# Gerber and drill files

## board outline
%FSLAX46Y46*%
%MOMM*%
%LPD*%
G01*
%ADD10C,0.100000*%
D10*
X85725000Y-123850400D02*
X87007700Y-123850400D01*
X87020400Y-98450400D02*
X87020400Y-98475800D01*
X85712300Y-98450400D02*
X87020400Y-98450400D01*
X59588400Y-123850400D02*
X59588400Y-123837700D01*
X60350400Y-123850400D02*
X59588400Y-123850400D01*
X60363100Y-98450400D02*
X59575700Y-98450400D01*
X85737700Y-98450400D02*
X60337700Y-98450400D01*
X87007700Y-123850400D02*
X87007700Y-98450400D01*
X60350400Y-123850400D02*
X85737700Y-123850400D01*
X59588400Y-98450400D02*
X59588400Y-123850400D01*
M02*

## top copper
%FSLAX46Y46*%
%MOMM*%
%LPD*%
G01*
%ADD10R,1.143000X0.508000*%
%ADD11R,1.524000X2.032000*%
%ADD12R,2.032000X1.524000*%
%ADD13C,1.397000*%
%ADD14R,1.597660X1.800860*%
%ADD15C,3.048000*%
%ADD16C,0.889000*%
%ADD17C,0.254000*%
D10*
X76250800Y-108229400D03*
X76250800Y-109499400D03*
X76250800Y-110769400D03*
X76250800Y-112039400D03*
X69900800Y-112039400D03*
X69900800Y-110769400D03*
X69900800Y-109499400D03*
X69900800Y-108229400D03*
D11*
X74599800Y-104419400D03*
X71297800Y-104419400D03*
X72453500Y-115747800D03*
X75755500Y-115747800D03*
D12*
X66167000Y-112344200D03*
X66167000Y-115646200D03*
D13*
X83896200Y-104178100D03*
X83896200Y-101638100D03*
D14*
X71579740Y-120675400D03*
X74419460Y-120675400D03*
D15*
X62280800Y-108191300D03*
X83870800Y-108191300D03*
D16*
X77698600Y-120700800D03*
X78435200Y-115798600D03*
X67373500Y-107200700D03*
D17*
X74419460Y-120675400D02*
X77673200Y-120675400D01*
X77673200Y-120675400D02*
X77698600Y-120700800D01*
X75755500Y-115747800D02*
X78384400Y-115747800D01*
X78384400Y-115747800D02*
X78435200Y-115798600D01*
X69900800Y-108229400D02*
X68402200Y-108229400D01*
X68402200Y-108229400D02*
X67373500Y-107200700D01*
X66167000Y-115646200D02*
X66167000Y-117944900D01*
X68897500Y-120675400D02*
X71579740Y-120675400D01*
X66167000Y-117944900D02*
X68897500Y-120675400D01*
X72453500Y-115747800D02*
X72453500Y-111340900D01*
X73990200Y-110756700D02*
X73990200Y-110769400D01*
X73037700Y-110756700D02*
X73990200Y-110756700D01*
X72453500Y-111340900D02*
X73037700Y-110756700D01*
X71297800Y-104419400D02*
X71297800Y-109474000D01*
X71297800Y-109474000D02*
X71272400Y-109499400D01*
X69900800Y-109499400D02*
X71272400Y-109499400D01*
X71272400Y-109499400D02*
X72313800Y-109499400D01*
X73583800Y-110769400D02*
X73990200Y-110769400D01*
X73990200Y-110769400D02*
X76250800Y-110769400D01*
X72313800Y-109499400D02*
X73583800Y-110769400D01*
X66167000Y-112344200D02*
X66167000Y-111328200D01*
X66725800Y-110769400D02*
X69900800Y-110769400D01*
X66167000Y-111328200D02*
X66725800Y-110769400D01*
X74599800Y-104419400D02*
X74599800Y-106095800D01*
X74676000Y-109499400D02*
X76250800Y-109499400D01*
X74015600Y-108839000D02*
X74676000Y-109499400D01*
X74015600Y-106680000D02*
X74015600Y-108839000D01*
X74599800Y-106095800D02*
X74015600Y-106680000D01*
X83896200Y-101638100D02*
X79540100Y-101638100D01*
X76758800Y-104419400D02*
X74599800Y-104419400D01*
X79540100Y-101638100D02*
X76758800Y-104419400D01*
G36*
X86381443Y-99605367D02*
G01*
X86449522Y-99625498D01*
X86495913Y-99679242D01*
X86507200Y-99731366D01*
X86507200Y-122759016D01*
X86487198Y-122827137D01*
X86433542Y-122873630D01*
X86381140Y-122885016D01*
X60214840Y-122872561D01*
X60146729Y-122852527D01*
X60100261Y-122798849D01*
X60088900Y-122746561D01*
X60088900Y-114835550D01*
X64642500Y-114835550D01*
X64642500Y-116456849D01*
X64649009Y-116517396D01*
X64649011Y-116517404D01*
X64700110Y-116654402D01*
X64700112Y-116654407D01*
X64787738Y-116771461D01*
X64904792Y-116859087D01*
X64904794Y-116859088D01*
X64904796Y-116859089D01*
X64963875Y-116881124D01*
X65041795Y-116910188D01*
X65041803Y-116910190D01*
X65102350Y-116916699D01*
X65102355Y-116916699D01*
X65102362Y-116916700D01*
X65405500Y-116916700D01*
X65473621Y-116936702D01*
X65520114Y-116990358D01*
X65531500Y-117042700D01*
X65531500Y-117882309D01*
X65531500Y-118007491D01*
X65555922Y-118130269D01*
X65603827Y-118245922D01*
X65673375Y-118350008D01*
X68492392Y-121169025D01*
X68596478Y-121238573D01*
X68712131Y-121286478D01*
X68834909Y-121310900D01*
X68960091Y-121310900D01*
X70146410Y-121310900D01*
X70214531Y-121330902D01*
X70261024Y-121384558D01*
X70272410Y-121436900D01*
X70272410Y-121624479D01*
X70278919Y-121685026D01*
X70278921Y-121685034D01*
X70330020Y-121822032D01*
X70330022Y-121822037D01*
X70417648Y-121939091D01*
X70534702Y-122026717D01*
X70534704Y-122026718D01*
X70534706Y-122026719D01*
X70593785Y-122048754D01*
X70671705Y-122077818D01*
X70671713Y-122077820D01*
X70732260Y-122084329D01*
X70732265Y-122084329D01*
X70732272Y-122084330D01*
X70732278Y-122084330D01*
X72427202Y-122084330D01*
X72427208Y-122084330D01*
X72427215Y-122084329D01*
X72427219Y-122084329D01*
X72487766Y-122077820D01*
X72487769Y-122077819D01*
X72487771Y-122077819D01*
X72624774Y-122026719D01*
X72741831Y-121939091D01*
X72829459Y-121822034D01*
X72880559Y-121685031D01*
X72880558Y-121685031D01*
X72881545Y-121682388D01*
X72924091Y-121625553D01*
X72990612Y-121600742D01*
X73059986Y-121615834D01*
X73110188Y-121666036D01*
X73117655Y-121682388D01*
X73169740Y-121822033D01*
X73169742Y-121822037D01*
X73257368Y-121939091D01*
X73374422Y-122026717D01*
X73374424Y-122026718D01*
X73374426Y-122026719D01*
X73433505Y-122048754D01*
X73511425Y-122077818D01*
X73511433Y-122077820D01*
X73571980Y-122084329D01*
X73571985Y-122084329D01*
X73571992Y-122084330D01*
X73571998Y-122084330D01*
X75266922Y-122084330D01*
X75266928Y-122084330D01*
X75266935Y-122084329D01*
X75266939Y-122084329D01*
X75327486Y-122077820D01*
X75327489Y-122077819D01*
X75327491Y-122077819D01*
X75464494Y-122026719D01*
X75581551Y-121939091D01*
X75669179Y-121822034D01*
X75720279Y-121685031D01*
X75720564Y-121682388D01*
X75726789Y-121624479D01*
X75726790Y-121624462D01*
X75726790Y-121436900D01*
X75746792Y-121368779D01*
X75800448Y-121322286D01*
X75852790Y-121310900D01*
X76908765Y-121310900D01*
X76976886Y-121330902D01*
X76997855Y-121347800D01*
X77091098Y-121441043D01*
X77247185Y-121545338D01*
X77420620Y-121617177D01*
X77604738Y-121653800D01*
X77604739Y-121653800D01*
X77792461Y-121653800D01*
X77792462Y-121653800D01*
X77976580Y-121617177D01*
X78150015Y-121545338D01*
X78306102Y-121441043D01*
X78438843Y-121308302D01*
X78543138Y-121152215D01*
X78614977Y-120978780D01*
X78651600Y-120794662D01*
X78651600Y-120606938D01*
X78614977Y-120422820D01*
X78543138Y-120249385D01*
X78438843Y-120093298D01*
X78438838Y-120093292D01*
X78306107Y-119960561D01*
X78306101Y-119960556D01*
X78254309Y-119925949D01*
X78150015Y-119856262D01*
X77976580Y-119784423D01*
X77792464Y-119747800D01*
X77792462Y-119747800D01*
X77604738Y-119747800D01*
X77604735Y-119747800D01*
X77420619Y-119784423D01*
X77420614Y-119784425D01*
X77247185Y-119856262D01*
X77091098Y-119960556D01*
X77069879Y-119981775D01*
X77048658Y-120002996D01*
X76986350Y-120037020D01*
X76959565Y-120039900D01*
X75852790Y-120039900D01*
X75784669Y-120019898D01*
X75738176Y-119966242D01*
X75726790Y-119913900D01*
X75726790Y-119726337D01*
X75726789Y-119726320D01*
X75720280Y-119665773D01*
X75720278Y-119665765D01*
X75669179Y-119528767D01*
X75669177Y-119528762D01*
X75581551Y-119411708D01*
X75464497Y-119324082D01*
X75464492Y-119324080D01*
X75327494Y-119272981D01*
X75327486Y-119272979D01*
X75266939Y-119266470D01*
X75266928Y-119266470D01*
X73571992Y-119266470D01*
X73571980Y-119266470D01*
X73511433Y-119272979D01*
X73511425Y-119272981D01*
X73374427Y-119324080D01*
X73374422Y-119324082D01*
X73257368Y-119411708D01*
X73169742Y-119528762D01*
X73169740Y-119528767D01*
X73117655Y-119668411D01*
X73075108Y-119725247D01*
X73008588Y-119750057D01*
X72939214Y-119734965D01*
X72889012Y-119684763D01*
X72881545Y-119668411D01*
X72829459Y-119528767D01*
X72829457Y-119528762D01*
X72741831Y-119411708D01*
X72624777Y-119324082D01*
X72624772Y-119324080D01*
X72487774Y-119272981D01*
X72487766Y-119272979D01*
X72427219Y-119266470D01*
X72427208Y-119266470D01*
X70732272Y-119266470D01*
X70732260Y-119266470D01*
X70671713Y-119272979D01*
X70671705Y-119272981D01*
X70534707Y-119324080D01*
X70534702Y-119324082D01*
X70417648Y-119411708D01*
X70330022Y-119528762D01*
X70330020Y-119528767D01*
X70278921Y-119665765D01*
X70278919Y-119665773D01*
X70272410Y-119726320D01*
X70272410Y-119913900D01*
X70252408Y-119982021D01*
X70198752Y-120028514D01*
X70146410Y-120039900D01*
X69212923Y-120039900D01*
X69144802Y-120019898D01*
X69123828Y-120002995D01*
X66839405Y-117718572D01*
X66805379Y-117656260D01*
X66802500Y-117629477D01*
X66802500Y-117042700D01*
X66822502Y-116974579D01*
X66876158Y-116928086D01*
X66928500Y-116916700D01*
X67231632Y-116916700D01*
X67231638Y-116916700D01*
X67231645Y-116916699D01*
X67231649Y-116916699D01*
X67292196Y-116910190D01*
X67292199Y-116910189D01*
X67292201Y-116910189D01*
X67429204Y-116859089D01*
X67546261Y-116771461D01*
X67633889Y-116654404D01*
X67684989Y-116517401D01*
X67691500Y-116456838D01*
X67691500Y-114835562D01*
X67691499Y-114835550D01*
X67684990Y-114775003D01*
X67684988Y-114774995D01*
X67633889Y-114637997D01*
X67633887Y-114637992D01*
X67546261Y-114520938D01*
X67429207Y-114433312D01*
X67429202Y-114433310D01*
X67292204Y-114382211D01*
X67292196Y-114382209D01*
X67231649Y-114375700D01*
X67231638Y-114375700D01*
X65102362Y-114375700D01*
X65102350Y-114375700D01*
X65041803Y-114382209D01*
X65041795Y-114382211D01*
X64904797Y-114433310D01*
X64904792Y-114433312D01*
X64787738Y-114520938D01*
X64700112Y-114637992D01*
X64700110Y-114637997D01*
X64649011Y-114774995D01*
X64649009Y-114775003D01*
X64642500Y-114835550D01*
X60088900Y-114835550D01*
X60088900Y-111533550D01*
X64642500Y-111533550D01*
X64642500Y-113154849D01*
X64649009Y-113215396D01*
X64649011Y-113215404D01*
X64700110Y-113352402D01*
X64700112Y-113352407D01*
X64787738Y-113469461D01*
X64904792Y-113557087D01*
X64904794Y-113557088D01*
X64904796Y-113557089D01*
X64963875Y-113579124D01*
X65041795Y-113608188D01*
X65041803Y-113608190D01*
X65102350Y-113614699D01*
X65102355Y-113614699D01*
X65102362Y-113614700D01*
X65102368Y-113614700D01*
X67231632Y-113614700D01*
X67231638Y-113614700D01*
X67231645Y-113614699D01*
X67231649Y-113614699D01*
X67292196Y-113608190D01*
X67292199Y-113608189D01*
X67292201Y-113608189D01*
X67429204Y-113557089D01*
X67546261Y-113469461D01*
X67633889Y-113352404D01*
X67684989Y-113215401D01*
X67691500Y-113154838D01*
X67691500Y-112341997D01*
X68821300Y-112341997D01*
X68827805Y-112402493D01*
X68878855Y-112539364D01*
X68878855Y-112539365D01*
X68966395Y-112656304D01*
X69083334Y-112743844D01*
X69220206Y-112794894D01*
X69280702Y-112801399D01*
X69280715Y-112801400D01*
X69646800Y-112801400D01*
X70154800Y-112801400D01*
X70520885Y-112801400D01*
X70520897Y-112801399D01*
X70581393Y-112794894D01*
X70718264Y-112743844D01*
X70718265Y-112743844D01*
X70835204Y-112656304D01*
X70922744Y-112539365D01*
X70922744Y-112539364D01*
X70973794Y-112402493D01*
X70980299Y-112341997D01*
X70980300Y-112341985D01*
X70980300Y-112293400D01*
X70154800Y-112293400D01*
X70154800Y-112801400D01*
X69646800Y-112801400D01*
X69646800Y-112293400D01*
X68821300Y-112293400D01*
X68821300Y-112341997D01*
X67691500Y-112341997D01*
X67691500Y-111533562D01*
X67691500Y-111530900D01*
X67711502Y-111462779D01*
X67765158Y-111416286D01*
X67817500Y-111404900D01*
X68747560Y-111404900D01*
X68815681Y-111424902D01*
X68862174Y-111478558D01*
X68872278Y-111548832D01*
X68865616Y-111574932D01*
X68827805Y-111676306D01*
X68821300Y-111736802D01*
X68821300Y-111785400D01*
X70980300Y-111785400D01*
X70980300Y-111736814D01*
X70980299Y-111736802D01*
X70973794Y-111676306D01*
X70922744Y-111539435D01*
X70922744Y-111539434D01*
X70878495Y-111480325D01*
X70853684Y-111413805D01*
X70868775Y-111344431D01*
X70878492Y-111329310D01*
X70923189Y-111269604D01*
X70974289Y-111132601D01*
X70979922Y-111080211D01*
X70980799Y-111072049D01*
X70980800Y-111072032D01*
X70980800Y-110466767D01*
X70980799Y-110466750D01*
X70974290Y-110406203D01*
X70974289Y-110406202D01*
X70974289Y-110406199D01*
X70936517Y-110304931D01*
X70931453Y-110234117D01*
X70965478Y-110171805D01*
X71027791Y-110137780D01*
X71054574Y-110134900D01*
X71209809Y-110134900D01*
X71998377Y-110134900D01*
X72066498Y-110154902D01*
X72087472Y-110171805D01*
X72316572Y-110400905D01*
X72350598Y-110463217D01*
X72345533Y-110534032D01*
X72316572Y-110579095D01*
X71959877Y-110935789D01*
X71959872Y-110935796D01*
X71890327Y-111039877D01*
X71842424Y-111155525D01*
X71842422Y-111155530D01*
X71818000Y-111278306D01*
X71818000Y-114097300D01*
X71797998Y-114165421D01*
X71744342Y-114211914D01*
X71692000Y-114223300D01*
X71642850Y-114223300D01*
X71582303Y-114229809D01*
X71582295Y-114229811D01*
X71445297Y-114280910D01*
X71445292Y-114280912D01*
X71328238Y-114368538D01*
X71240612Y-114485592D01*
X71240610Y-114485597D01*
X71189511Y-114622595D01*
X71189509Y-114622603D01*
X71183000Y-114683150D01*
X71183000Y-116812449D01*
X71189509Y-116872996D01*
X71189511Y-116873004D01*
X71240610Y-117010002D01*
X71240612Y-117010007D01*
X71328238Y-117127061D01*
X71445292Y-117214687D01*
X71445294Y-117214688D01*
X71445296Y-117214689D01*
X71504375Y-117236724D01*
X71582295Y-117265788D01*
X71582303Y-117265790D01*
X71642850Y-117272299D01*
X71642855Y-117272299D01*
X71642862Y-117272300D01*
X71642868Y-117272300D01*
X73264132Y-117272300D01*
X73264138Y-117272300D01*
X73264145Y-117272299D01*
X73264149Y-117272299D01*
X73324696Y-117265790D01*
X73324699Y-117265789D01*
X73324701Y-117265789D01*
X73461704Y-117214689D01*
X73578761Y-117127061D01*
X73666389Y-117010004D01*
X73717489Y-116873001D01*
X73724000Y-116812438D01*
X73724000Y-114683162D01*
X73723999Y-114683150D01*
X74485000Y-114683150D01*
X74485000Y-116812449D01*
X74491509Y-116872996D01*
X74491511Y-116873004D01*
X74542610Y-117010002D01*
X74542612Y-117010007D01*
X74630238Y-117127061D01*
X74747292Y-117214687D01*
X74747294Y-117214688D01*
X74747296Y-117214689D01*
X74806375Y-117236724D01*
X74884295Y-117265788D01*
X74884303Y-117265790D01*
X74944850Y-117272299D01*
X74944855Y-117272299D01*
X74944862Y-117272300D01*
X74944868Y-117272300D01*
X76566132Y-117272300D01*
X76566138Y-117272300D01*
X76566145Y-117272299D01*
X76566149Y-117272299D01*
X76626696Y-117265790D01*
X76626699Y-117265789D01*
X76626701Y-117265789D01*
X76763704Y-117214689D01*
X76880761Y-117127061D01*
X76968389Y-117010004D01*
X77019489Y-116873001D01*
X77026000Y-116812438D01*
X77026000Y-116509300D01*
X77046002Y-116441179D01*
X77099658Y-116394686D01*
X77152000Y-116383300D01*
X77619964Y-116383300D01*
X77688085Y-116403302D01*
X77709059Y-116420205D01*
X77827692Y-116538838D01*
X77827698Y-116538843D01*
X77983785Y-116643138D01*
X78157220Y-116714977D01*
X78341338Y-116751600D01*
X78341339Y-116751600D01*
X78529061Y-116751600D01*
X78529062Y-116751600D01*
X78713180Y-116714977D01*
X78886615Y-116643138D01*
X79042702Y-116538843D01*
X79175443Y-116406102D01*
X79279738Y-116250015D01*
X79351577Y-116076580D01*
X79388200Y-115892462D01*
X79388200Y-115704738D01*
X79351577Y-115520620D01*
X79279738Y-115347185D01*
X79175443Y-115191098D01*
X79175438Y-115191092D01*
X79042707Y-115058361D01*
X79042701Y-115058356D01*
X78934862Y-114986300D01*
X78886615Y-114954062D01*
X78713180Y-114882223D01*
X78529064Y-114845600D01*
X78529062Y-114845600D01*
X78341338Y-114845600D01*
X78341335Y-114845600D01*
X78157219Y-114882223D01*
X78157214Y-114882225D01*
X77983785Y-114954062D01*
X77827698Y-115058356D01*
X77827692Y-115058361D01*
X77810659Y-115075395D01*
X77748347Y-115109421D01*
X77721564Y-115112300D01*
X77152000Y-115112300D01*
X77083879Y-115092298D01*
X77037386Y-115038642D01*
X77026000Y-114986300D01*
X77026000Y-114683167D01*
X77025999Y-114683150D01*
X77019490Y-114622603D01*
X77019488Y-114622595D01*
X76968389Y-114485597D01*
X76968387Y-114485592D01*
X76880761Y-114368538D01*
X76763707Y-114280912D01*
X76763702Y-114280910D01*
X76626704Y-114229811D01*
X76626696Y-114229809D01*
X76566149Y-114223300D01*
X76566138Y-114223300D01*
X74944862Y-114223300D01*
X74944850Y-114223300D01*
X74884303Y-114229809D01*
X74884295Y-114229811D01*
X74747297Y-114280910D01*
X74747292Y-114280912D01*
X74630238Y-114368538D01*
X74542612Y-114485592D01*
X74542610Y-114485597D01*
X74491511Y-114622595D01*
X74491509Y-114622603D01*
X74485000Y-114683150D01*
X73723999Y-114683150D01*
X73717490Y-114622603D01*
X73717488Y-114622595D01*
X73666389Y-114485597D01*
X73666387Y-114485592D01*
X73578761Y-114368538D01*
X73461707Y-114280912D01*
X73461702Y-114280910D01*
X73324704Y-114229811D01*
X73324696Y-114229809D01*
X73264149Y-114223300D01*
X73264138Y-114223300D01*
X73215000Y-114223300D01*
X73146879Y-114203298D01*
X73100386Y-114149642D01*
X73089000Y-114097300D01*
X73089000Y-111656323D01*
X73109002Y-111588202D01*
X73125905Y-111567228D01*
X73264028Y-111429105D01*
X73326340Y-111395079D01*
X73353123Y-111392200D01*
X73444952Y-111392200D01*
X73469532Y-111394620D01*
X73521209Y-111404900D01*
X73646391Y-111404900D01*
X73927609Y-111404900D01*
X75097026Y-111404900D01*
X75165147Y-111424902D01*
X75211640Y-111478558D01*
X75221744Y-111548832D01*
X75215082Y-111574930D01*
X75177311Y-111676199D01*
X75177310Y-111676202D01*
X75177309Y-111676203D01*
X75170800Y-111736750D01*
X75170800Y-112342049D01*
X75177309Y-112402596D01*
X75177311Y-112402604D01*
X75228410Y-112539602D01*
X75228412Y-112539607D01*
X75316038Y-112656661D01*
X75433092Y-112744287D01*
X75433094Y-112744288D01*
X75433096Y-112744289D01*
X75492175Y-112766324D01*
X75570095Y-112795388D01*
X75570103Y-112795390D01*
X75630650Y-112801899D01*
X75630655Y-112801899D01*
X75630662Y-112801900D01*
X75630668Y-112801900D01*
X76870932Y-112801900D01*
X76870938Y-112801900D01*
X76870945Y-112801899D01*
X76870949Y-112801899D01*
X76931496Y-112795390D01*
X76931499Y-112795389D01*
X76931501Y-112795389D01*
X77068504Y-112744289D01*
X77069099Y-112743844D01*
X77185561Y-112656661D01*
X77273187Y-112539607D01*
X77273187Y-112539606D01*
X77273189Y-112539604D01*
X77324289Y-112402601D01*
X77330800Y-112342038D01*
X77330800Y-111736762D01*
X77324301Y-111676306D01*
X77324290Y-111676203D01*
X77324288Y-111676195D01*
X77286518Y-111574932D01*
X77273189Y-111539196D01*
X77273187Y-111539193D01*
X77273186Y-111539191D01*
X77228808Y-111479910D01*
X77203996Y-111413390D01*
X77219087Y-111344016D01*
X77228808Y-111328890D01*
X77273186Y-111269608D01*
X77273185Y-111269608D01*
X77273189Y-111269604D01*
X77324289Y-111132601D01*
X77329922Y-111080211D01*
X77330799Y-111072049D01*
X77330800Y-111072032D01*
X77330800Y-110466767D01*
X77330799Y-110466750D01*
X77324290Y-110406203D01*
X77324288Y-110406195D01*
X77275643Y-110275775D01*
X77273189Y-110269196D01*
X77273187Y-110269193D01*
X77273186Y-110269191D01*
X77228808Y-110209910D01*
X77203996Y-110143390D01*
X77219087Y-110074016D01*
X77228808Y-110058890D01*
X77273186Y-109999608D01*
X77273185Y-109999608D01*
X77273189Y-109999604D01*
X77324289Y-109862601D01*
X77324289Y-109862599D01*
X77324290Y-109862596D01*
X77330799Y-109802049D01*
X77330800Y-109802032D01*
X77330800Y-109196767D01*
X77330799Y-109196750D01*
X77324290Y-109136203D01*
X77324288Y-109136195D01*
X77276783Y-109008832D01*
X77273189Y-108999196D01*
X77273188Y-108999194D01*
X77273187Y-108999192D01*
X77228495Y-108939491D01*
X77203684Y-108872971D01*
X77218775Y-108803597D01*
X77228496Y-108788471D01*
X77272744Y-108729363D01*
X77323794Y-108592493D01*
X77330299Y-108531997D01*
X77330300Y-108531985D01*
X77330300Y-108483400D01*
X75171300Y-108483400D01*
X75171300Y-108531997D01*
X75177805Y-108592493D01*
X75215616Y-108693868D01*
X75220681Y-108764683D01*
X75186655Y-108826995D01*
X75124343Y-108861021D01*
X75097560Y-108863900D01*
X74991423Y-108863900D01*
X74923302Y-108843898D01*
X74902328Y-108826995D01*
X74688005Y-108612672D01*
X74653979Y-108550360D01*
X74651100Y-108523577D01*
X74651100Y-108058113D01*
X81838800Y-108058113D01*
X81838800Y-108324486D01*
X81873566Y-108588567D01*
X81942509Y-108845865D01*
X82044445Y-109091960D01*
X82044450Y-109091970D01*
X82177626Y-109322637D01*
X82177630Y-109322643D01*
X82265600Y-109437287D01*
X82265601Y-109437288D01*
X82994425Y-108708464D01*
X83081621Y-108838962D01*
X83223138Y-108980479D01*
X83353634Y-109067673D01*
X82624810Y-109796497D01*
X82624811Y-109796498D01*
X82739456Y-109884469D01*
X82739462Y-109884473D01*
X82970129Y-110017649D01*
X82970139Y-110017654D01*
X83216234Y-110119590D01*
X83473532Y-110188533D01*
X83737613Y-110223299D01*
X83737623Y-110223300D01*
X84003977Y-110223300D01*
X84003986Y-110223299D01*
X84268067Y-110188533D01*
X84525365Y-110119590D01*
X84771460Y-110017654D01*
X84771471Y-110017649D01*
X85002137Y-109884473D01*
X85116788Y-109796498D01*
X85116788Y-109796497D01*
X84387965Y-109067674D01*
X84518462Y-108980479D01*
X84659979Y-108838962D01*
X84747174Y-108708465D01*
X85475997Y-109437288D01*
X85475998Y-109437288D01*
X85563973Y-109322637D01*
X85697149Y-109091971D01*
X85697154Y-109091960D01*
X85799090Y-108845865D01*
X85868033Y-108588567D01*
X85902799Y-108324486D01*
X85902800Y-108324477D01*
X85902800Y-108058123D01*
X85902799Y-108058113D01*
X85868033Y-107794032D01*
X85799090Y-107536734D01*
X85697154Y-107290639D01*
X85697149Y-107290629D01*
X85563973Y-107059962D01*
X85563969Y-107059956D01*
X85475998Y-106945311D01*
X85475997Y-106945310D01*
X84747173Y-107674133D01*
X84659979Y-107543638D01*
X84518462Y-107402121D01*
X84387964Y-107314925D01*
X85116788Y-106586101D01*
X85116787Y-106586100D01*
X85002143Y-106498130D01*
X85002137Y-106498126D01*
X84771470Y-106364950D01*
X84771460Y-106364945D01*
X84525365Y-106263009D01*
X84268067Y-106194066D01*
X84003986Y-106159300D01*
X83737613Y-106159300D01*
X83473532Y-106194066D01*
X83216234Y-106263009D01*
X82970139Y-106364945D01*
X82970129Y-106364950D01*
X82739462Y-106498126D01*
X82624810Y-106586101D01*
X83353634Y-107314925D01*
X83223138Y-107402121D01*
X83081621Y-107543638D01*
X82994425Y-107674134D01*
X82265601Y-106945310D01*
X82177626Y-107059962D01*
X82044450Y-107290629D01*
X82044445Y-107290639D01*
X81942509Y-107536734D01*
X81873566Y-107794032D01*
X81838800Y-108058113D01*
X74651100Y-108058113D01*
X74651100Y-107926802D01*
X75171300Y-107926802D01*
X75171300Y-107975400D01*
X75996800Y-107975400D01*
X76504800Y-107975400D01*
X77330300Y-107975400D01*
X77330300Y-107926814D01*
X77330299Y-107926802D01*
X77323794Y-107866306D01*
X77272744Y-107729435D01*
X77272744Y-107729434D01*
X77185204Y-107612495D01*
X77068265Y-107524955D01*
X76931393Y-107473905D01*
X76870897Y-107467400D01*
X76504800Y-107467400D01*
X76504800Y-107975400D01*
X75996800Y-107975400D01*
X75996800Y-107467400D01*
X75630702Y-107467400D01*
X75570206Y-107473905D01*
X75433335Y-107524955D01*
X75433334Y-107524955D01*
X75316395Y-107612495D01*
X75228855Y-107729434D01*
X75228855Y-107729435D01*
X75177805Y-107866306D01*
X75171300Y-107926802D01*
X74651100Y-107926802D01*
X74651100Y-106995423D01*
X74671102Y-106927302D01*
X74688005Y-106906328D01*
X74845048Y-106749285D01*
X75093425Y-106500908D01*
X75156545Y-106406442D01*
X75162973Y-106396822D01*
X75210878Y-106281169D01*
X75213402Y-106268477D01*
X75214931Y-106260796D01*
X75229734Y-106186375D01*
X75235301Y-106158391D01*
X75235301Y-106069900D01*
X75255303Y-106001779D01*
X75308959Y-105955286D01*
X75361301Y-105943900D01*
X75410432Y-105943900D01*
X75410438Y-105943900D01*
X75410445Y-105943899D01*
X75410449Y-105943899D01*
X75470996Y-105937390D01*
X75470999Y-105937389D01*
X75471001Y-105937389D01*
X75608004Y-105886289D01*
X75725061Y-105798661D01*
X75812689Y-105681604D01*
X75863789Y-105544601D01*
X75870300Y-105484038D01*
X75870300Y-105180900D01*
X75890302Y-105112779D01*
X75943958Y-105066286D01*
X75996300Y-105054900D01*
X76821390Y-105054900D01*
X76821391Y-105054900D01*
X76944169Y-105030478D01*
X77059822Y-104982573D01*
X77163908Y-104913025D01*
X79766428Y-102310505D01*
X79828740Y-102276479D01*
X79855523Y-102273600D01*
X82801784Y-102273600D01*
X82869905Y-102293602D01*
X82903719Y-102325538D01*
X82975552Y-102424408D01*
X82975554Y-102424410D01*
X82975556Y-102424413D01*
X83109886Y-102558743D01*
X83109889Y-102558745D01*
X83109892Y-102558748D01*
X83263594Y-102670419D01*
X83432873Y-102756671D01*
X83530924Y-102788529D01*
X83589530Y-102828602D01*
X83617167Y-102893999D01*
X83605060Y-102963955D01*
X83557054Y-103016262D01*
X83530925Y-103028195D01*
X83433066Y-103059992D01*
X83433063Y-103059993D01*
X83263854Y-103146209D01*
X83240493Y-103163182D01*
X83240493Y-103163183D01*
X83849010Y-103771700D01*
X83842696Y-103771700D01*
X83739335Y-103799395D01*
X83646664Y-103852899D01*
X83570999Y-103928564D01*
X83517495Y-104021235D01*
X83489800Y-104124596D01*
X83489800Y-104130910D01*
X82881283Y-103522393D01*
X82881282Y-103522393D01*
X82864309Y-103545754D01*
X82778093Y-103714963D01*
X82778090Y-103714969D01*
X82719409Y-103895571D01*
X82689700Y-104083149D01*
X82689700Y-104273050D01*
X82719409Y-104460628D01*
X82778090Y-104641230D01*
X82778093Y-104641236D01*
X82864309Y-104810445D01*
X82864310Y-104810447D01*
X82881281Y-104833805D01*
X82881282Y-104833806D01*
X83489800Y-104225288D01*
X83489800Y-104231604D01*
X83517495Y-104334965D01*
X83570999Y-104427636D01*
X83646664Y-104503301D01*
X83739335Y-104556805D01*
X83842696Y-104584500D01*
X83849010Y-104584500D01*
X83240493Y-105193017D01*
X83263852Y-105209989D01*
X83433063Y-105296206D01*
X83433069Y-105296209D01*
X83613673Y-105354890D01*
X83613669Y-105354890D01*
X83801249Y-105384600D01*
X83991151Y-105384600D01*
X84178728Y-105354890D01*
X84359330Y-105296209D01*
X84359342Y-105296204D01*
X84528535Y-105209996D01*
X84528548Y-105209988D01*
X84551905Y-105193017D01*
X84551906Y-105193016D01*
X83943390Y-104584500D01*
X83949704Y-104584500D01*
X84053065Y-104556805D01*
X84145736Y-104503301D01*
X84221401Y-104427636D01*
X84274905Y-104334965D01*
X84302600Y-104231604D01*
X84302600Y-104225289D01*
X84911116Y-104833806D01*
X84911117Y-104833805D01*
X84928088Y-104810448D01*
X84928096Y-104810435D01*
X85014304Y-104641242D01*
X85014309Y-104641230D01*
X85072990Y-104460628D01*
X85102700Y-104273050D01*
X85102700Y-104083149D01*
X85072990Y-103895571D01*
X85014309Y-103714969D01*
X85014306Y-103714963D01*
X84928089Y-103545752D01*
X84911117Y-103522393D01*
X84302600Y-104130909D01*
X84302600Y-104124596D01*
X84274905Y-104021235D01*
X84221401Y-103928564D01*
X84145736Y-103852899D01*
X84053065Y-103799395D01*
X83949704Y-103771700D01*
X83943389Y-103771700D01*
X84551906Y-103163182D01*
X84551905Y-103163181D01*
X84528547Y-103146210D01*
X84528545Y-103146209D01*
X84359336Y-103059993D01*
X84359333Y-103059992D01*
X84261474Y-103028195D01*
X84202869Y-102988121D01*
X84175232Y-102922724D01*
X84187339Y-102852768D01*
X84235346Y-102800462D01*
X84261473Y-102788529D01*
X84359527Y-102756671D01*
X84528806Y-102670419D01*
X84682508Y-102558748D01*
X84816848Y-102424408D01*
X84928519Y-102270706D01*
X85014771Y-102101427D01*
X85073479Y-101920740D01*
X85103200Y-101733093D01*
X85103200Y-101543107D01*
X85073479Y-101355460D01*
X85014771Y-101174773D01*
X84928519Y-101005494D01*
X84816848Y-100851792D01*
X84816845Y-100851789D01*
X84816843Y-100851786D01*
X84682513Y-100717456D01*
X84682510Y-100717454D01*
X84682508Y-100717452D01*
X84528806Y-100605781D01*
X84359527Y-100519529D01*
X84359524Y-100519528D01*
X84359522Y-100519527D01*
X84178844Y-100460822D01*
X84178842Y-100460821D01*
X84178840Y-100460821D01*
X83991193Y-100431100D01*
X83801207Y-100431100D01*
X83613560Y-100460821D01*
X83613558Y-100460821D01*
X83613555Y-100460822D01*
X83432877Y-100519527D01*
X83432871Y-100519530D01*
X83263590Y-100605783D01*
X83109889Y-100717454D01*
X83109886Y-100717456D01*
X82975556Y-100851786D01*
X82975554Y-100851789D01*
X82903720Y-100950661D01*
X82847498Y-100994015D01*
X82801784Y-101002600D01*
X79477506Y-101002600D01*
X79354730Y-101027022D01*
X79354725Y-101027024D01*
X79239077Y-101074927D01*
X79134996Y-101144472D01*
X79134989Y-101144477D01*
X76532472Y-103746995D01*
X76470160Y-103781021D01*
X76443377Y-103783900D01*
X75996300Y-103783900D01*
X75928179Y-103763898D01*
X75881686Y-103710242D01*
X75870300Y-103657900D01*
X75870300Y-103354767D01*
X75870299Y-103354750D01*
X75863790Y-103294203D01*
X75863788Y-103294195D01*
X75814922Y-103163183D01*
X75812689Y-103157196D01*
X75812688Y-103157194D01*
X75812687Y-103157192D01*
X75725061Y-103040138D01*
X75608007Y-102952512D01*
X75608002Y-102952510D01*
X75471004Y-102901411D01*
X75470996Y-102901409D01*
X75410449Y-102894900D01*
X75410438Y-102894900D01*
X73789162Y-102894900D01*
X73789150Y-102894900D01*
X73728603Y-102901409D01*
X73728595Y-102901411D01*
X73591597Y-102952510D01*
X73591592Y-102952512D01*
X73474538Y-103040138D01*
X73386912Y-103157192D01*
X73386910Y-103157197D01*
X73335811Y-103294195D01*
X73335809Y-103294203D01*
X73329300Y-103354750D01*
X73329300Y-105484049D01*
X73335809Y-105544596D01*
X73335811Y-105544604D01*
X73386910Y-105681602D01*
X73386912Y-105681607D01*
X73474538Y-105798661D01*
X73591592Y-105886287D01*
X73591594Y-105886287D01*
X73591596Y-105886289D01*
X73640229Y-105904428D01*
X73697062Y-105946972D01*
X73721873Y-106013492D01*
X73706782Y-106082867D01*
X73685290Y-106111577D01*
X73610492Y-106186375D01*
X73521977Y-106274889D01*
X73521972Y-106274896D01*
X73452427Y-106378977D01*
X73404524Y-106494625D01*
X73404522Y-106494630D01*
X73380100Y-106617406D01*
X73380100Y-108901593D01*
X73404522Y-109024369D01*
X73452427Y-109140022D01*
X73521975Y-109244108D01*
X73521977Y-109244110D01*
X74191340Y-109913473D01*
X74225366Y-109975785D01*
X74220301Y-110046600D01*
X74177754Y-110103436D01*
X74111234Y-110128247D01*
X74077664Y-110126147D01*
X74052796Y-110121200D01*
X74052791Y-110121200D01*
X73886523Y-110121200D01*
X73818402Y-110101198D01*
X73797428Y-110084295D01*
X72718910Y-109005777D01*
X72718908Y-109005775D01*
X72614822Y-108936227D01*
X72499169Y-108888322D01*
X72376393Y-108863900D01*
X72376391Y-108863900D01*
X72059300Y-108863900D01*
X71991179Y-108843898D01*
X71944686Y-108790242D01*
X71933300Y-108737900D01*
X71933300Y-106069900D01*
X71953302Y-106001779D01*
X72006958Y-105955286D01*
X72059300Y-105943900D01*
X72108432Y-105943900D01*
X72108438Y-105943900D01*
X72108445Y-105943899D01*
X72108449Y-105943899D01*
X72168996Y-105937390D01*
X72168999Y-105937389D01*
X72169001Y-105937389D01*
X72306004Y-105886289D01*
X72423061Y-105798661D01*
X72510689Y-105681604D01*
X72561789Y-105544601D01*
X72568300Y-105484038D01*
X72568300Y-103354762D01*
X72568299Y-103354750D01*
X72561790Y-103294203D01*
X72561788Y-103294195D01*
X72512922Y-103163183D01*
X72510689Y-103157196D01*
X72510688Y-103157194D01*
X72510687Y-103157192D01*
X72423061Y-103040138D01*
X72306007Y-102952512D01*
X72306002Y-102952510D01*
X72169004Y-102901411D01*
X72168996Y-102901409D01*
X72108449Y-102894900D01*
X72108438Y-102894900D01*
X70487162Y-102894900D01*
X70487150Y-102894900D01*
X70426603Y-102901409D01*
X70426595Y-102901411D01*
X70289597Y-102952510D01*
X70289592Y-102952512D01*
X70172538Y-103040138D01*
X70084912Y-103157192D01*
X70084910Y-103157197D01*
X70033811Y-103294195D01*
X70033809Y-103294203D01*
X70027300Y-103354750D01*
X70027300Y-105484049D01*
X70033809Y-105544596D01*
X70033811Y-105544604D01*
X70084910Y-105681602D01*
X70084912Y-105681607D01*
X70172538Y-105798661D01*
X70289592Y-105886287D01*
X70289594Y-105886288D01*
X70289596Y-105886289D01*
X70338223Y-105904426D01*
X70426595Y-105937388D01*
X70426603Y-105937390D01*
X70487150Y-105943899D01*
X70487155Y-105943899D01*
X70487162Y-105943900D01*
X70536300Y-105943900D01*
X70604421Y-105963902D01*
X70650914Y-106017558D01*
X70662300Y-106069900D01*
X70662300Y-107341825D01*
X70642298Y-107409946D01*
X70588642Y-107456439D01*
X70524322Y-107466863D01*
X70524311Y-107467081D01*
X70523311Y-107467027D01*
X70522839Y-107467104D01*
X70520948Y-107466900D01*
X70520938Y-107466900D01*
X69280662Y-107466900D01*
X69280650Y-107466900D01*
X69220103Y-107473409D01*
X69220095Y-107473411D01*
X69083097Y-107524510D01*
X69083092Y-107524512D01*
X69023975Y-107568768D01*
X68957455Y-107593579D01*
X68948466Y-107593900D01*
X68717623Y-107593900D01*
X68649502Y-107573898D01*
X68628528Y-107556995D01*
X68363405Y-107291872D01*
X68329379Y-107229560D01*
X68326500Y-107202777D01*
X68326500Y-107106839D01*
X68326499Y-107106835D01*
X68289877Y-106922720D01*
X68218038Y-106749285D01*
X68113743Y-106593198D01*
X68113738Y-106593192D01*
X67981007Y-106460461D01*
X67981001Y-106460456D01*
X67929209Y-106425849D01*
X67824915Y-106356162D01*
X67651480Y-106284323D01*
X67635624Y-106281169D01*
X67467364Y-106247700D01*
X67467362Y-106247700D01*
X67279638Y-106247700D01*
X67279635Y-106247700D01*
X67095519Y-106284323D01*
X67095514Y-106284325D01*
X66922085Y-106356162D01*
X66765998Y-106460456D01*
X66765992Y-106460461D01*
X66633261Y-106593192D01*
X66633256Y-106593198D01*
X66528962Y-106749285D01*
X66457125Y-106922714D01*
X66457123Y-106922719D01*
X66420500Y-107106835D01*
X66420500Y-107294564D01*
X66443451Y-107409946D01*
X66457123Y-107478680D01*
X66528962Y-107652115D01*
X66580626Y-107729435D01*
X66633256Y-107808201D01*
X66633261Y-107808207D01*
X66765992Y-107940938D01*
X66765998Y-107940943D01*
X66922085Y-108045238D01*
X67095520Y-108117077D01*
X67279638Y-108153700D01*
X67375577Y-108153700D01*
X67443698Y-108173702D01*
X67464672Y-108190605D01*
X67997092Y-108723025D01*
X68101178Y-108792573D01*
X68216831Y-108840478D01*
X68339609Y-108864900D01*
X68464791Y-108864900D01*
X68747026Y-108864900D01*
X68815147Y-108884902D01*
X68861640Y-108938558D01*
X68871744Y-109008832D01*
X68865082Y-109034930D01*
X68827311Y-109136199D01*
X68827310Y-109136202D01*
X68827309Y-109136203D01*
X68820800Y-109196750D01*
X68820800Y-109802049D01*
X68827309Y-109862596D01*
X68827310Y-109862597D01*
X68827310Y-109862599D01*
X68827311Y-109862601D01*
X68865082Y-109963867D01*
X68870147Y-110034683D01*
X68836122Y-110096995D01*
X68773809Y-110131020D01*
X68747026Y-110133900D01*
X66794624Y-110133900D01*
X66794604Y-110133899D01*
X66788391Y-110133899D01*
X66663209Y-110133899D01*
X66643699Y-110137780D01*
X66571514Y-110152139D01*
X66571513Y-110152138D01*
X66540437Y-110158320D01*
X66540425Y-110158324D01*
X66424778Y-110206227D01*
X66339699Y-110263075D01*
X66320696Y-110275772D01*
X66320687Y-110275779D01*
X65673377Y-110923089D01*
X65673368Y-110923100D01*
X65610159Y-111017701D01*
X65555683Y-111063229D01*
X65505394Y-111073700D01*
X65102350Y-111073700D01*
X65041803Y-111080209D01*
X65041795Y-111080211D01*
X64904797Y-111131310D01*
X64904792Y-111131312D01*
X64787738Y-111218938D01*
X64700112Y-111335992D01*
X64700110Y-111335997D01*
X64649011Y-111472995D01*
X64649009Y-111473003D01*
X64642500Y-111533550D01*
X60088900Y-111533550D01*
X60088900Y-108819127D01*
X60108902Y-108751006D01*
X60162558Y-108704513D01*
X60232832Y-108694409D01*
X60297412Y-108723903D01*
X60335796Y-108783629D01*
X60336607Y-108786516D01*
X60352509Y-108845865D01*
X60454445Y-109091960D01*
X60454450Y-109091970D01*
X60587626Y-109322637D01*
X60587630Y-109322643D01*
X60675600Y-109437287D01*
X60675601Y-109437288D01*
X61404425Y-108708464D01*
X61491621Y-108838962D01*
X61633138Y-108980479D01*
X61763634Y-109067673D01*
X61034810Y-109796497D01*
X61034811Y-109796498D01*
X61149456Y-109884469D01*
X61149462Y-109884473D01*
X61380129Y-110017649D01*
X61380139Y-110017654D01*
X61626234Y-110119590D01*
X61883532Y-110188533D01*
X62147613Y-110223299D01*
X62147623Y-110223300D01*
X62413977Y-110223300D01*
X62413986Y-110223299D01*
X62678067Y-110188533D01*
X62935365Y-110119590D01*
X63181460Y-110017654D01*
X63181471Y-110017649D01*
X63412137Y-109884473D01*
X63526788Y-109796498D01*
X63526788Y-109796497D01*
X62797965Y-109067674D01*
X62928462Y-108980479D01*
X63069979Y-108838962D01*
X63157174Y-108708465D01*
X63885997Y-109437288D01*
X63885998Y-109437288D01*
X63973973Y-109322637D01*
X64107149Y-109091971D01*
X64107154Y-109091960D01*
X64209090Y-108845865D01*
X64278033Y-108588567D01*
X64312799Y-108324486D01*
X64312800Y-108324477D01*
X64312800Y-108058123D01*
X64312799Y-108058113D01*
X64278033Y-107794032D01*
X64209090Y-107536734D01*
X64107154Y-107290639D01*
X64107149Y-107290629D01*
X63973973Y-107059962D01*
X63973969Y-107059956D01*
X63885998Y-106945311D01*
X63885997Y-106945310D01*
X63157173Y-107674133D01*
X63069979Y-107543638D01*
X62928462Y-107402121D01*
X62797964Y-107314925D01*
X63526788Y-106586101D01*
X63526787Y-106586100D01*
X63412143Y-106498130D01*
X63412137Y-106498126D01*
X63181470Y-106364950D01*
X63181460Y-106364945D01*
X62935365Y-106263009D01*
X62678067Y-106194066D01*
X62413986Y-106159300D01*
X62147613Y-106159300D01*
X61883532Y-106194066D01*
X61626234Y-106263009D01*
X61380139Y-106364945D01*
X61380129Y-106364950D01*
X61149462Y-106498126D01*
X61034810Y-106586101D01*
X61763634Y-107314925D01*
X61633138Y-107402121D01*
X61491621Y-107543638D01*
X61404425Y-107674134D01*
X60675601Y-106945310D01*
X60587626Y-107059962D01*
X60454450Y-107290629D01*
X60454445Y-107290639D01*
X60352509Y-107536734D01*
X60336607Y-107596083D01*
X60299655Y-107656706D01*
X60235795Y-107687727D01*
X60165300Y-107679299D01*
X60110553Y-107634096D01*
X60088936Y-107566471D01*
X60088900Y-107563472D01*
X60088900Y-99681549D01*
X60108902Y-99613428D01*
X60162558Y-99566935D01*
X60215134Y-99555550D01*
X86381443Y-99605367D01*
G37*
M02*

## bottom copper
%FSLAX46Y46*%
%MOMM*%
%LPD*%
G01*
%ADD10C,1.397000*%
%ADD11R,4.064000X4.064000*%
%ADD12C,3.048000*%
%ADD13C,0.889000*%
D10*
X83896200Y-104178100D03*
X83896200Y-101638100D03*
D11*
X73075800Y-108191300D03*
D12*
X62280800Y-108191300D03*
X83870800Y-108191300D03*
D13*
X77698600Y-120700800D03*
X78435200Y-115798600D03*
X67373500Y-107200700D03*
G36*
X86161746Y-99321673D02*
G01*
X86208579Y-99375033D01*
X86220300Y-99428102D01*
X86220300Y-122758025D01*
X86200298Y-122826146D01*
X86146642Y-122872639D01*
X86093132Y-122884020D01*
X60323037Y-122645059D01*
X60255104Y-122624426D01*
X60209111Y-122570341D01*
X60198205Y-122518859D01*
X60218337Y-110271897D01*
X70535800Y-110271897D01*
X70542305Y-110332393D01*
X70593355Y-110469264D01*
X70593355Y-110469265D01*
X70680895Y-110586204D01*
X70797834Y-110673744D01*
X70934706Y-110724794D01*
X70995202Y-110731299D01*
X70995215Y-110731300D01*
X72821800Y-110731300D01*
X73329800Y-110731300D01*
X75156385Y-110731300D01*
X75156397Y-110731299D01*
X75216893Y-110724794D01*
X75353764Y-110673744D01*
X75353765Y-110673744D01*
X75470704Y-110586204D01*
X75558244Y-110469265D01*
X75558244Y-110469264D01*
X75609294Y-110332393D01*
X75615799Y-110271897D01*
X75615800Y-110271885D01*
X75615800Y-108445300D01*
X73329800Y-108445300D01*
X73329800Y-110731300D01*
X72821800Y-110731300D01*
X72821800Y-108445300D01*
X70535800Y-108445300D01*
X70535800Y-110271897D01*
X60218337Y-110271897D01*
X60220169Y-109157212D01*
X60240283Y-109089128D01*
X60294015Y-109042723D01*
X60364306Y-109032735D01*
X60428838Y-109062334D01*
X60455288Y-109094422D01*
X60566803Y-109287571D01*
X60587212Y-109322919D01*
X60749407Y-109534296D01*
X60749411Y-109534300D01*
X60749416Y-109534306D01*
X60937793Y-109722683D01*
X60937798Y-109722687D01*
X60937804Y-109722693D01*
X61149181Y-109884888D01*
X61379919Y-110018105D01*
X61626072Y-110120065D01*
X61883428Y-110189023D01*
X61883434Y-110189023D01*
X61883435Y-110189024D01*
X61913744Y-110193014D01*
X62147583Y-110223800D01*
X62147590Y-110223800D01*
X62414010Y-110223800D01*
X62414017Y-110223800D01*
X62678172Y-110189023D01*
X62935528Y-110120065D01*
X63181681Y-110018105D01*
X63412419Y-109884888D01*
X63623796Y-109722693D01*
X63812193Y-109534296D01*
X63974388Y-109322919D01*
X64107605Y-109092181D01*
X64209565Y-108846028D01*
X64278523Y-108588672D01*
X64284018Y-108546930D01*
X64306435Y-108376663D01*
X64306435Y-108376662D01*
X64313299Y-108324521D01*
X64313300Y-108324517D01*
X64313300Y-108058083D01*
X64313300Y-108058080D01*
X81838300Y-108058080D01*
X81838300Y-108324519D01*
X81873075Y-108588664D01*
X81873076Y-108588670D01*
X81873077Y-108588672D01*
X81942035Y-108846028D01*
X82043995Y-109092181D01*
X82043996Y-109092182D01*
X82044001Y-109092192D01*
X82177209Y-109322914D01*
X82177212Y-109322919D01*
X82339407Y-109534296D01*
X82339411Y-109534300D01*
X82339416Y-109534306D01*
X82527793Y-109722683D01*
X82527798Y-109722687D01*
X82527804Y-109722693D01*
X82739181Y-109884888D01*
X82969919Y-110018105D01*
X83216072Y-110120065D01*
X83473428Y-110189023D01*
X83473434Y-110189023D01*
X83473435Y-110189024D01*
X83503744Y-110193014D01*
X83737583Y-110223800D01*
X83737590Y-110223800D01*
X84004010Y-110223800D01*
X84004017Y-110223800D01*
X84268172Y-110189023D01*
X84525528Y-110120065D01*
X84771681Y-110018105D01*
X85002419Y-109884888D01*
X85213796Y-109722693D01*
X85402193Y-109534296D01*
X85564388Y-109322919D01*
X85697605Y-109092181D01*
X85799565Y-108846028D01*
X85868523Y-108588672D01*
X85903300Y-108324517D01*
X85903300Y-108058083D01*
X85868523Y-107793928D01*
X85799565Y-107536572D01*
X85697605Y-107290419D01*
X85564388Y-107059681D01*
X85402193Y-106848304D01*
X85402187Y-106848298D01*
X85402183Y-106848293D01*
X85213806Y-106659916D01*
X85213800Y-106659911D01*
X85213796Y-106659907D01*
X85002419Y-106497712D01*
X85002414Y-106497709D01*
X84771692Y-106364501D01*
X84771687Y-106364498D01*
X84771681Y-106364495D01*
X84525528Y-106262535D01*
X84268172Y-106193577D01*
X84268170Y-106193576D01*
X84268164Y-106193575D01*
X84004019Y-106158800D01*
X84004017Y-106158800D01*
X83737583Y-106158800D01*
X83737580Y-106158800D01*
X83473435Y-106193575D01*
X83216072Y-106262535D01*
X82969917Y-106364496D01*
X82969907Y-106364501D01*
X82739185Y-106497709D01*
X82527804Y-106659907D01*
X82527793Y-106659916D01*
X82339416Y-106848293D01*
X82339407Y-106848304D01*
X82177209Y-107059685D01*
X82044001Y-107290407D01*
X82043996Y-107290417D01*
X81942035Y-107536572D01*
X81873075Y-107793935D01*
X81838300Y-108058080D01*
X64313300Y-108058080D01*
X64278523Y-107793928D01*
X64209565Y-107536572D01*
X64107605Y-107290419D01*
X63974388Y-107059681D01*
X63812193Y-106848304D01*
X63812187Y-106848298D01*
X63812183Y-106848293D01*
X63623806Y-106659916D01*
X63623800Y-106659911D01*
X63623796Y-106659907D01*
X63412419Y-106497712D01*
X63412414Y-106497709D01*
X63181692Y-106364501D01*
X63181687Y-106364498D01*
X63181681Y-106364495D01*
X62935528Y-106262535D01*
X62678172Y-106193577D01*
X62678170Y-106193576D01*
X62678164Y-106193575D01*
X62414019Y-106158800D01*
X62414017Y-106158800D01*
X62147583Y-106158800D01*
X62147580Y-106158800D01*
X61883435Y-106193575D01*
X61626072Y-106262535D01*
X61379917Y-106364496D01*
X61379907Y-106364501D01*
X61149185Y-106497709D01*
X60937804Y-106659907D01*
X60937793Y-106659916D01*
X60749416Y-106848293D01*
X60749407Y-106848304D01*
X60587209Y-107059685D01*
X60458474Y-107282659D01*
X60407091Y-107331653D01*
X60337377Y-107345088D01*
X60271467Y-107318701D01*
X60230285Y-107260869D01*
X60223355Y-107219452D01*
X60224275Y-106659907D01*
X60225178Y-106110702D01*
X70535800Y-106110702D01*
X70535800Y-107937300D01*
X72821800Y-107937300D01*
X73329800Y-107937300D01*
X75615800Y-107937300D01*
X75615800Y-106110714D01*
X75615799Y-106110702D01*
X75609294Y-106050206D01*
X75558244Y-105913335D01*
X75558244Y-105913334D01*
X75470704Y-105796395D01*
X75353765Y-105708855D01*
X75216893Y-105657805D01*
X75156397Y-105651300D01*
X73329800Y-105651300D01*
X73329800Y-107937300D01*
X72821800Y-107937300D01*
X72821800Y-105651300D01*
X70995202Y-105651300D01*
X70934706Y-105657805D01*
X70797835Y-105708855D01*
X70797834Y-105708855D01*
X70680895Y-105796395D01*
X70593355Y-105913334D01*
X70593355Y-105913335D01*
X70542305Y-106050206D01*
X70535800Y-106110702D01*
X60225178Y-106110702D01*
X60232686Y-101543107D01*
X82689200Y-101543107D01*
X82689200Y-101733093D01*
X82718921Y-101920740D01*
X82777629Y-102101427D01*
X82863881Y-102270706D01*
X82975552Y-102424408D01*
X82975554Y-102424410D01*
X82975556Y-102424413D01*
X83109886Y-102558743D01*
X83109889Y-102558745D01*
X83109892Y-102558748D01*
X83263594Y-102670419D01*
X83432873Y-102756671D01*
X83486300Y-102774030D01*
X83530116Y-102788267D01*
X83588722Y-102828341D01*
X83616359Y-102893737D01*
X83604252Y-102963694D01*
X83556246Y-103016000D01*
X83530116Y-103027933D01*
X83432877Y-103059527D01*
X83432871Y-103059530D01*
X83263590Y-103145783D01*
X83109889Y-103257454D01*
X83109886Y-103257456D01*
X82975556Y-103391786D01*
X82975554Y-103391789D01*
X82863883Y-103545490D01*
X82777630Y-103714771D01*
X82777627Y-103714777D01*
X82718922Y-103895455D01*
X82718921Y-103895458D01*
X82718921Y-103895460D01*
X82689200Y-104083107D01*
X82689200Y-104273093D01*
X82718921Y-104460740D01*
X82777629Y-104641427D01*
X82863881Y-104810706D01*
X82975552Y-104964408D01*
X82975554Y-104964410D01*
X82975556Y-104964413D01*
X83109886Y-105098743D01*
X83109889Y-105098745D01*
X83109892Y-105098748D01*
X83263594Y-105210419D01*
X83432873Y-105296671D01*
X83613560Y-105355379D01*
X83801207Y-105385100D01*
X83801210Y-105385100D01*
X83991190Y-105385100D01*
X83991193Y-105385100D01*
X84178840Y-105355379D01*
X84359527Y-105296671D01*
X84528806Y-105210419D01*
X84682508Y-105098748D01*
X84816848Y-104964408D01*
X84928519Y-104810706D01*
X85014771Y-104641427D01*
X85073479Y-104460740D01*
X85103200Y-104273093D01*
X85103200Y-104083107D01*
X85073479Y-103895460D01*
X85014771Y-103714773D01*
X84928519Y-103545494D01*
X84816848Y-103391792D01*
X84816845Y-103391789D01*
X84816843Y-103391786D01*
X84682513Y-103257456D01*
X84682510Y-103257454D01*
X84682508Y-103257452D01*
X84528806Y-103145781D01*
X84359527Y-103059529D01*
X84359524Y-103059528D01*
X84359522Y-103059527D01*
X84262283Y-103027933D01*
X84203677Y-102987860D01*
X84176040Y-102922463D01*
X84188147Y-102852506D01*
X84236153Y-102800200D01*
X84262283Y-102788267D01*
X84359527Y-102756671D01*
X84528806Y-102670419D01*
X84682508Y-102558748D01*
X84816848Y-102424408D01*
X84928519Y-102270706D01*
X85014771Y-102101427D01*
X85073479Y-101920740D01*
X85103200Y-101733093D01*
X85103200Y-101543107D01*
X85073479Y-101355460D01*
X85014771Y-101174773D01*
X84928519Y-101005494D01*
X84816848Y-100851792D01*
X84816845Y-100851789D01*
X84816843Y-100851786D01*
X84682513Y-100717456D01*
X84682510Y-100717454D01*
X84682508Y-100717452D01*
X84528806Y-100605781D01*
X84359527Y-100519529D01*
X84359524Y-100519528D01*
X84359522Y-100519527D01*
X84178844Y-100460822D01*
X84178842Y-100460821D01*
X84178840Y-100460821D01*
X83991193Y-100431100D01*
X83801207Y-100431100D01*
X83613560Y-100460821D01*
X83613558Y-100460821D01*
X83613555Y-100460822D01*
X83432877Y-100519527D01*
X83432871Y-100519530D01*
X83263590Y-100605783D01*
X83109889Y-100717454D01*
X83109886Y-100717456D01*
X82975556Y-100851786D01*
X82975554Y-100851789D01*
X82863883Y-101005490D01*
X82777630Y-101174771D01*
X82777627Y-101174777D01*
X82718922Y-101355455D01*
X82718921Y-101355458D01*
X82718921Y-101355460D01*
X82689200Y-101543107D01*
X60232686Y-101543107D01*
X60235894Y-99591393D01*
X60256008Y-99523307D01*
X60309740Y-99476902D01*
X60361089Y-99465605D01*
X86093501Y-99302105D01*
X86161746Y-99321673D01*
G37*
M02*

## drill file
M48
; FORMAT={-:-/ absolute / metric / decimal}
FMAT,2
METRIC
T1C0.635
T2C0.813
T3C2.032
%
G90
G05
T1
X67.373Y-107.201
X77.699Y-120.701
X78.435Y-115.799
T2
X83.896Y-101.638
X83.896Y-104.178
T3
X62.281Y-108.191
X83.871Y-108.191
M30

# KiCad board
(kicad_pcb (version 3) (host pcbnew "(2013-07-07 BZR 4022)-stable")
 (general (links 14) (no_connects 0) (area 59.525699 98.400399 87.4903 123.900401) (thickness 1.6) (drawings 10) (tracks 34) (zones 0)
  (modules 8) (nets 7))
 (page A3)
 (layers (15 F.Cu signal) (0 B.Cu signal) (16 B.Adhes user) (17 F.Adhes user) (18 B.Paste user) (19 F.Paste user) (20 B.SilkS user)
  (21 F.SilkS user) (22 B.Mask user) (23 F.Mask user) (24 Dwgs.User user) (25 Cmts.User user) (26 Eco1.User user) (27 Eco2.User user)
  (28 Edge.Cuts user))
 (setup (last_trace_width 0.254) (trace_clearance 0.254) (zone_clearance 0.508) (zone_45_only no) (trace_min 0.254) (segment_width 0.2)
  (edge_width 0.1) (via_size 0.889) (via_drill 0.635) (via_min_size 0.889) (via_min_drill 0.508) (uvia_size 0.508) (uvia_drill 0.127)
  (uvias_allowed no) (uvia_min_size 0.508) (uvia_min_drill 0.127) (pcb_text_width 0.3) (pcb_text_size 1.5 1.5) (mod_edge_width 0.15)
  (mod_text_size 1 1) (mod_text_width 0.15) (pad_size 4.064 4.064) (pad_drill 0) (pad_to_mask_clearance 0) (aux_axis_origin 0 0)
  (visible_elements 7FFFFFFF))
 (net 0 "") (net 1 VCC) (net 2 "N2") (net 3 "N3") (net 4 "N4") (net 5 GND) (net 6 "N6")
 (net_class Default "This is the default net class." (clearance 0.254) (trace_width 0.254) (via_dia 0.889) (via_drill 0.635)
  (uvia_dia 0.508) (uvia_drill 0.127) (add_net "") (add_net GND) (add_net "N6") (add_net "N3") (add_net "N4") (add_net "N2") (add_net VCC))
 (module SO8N (layer F.Cu) (at 73.0758 110.1344 270)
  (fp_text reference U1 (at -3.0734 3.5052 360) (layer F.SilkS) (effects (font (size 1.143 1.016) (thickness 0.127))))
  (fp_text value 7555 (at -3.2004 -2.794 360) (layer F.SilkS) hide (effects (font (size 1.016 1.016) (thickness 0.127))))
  (pad 8 smd rect (at -1.905 -3.175 270) (size 0.508 1.143) (layers F.Cu F.Paste F.Mask) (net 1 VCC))
  (pad 7 smd rect (at -0.635 -3.175 270) (size 0.508 1.143) (layers F.Cu F.Paste F.Mask) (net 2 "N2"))
  (pad 6 smd rect (at 0.635 -3.175 270) (size 0.508 1.143) (layers F.Cu F.Paste F.Mask) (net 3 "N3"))
  (pad 5 smd rect (at 1.905 -3.175 270) (size 0.508 1.143) (layers F.Cu F.Paste F.Mask))
  (pad 4 smd rect (at 1.905 3.175 270) (size 0.508 1.143) (layers F.Cu F.Paste F.Mask) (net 1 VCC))
  (pad 3 smd rect (at 0.635 3.175 270) (size 0.508 1.143) (layers F.Cu F.Paste F.Mask) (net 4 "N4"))
  (pad 2 smd rect (at -0.635 3.175 270) (size 0.508 1.143) (layers F.Cu F.Paste F.Mask) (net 3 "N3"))
  (pad 1 smd rect (at -1.905 3.175 270) (size 0.508 1.143) (layers F.Cu F.Paste F.Mask) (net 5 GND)))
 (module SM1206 (layer F.Cu) (at 72.9488 104.4194 180)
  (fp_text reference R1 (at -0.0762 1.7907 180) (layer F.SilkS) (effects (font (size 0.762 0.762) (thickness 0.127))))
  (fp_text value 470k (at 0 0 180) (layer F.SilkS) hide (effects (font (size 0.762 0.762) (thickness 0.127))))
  (pad 1 smd rect (at -1.651 0 180) (size 1.524 2.032) (layers F.Cu F.Paste F.Mask) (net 2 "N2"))
  (pad 2 smd rect (at 1.651 0 180) (size 1.524 2.032) (layers F.Cu F.Paste F.Mask) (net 3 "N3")))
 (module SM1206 (layer F.Cu) (at 74.1045 115.7478)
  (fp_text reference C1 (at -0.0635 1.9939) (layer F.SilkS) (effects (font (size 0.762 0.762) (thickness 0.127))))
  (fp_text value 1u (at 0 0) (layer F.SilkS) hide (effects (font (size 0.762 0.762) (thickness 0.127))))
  (pad 1 smd rect (at -1.651 0) (size 1.524 2.032) (layers F.Cu F.Paste F.Mask) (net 3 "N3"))
  (pad 2 smd rect (at 1.651 0) (size 1.524 2.032) (layers F.Cu F.Paste F.Mask) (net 5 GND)))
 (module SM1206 (layer F.Cu) (at 66.167 113.9952 270)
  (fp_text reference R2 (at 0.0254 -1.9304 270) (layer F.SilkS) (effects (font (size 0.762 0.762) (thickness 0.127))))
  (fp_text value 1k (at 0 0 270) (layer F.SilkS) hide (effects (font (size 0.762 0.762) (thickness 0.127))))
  (pad 1 smd rect (at -1.651 0 270) (size 1.524 2.032) (layers F.Cu F.Paste F.Mask) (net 4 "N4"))
  (pad 2 smd rect (at 1.651 0 270) (size 1.524 2.032) (layers F.Cu F.Paste F.Mask) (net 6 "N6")))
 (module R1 (layer F.Cu) (at 83.8962 102.9081 90) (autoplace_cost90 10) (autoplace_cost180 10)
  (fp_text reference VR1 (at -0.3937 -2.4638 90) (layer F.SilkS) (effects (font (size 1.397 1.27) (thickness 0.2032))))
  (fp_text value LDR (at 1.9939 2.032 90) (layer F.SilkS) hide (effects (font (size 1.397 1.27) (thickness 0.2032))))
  (pad 1 thru_hole circle (at -1.27 0 90) (size 1.397 1.397) (drill 0.8128) (layers *.Cu *.Mask F.SilkS) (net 1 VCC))
  (pad 2 thru_hole circle (at 1.27 0 90) (size 1.397 1.397) (drill 0.8128) (layers *.Cu *.Mask F.SilkS) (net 2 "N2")))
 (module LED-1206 (layer F.Cu) (at 72.9996 120.6754)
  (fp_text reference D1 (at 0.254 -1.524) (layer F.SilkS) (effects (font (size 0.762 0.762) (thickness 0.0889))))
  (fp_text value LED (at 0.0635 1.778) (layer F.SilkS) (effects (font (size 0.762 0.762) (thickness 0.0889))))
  (pad 1 smd rect (at -1.41986 0) (size 1.59766 1.80086) (layers F.Cu F.Paste F.Mask) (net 6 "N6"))
  (pad 2 smd rect (at 1.41986 0) (size 1.59766 1.80086) (layers F.Cu F.Paste F.Mask) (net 5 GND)))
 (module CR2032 (layer B.Cu) (at 73.0758 108.1913 180)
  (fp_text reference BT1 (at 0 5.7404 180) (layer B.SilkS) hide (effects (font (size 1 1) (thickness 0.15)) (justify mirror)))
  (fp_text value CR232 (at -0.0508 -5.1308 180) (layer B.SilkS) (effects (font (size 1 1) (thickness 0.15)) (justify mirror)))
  (pad 2 smd rect (at 0 0 180) (size 4.064 4.064) (layers B.Cu B.Paste B.Mask) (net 5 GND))
  (pad 1 thru_hole circle (at 10.795 0 180) (size 3.048 3.048) (drill 2.032) (layers *.Cu *.Mask B.SilkS) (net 1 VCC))
  (pad 1 thru_hole circle (at -10.795 0 180) (size 3.048 3.048) (drill 2.032) (layers *.Cu *.Mask B.SilkS) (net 1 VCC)))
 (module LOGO (layer F.Cu) (at 83.5914 120.3706)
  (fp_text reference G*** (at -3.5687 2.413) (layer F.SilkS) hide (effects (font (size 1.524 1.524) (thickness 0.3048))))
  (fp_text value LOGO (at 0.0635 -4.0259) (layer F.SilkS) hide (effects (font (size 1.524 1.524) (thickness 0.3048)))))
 (gr_line (start 85.725 123.8504) (end 87.0077 123.8504) (angle 90) (layer Edge.Cuts) (width 0.1))
 (gr_line (start 87.0204 98.4504) (end 87.0204 98.4758) (angle 90) (layer Edge.Cuts) (width 0.1))
 (gr_line (start 85.7123 98.4504) (end 87.0204 98.4504) (angle 90) (layer Edge.Cuts) (width 0.1))
 (gr_line (start 59.5884 123.8504) (end 59.5884 123.8377) (angle 90) (layer Edge.Cuts) (width 0.1))
 (gr_line (start 60.3504 123.8504) (end 59.5884 123.8504) (angle 90) (layer Edge.Cuts) (width 0.1))
 (gr_line (start 60.3631 98.4504) (end 59.5757 98.4504) (angle 90) (layer Edge.Cuts) (width 0.1))
 (gr_line (start 85.7377 98.4504) (end 60.3377 98.4504) (angle 90) (layer Edge.Cuts) (width 0.1))
 (gr_line (start 87.0077 123.8504) (end 87.0077 98.4504) (angle 90) (layer Edge.Cuts) (width 0.1))
 (gr_line (start 60.3504 123.8504) (end 85.7377 123.8504) (angle 90) (layer Edge.Cuts) (width 0.1))
 (gr_line (start 59.5884 98.4504) (end 59.5884 123.8504) (angle 90) (layer Edge.Cuts) (width 0.1))
 (segment (start 74.41946 120.6754) (end 77.6732 120.6754) (width 0.254) (layer F.Cu) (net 5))
 (via (at 77.6986 120.7008) (size 0.889) (layers F.Cu B.Cu) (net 5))
 (segment (start 77.6732 120.6754) (end 77.6986 120.7008) (width 0.254) (layer F.Cu) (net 5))
 (segment (start 75.7555 115.7478) (end 78.3844 115.7478) (width 0.254) (layer F.Cu) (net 5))
 (via (at 78.4352 115.7986) (size 0.889) (layers F.Cu B.Cu) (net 5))
 (segment (start 78.3844 115.7478) (end 78.4352 115.7986) (width 0.254) (layer F.Cu) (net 5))
 (segment (start 69.9008 108.2294) (end 68.4022 108.2294) (width 0.254) (layer F.Cu) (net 5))
 (via (at 67.3735 107.2007) (size 0.889) (layers F.Cu B.Cu) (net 5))
 (segment (start 68.4022 108.2294) (end 67.3735 107.2007) (width 0.254) (layer F.Cu) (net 5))
 (segment (start 66.167 115.6462) (end 66.167 117.9449) (width 0.254) (layer F.Cu) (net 6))
 (segment (start 68.8975 120.6754) (end 71.57974 120.6754) (width 0.254) (layer F.Cu) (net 6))
 (segment (start 66.167 117.9449) (end 68.8975 120.6754) (width 0.254) (layer F.Cu) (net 6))
 (segment (start 72.4535 115.7478) (end 72.4535 111.3409) (width 0.254) (layer F.Cu) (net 3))
 (segment (start 73.9902 110.7567) (end 73.9902 110.7694) (width 0.254) (layer F.Cu) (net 3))
 (segment (start 73.0377 110.7567) (end 73.9902 110.7567) (width 0.254) (layer F.Cu) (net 3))
 (segment (start 72.4535 111.3409) (end 73.0377 110.7567) (width 0.254) (layer F.Cu) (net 3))
 (segment (start 71.2978 104.4194) (end 71.2978 109.474) (width 0.254) (layer F.Cu) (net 3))
 (segment (start 71.2978 109.474) (end 71.2724 109.4994) (width 0.254) (layer F.Cu) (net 3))
 (segment (start 69.9008 109.4994) (end 71.2724 109.4994) (width 0.254) (layer F.Cu) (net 3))
 (segment (start 71.2724 109.4994) (end 72.3138 109.4994) (width 0.254) (layer F.Cu) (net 3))
 (segment (start 73.5838 110.7694) (end 73.9902 110.7694) (width 0.254) (layer F.Cu) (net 3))
 (segment (start 73.9902 110.7694) (end 76.2508 110.7694) (width 0.254) (layer F.Cu) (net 3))
 (segment (start 72.3138 109.4994) (end 73.5838 110.7694) (width 0.254) (layer F.Cu) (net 3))
 (segment (start 66.167 112.3442) (end 66.167 111.3282) (width 0.254) (layer F.Cu) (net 4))
 (segment (start 66.7258 110.7694) (end 69.9008 110.7694) (width 0.254) (layer F.Cu) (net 4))
 (segment (start 66.167 111.3282) (end 66.7258 110.7694) (width 0.254) (layer F.Cu) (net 4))
 (segment (start 74.5998 104.4194) (end 74.5998 106.0958) (width 0.254) (layer F.Cu) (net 2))
 (segment (start 74.676 109.4994) (end 76.2508 109.4994) (width 0.254) (layer F.Cu) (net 2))
 (segment (start 74.0156 108.839) (end 74.676 109.4994) (width 0.254) (layer F.Cu) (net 2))
 (segment (start 74.0156 106.68) (end 74.0156 108.839) (width 0.254) (layer F.Cu) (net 2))
 (segment (start 74.5998 106.0958) (end 74.0156 106.68) (width 0.254) (layer F.Cu) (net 2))
 (segment (start 83.8962 101.6381) (end 79.5401 101.6381) (width 0.254) (layer F.Cu) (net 2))
 (segment (start 76.7588 104.4194) (end 74.5998 104.4194) (width 0.254) (layer F.Cu) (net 2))
 (segment (start 79.5401 101.6381) (end 76.7588 104.4194) (width 0.254) (layer F.Cu) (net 2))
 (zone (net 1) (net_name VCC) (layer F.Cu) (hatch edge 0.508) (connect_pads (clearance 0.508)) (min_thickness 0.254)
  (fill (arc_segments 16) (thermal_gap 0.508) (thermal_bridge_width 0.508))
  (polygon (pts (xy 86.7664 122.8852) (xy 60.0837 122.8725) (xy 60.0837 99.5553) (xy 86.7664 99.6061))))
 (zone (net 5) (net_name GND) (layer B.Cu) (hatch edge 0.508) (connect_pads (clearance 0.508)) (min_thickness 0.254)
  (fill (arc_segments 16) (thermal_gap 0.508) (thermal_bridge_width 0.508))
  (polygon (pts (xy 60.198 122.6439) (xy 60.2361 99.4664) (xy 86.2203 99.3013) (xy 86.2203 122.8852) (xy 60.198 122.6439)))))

